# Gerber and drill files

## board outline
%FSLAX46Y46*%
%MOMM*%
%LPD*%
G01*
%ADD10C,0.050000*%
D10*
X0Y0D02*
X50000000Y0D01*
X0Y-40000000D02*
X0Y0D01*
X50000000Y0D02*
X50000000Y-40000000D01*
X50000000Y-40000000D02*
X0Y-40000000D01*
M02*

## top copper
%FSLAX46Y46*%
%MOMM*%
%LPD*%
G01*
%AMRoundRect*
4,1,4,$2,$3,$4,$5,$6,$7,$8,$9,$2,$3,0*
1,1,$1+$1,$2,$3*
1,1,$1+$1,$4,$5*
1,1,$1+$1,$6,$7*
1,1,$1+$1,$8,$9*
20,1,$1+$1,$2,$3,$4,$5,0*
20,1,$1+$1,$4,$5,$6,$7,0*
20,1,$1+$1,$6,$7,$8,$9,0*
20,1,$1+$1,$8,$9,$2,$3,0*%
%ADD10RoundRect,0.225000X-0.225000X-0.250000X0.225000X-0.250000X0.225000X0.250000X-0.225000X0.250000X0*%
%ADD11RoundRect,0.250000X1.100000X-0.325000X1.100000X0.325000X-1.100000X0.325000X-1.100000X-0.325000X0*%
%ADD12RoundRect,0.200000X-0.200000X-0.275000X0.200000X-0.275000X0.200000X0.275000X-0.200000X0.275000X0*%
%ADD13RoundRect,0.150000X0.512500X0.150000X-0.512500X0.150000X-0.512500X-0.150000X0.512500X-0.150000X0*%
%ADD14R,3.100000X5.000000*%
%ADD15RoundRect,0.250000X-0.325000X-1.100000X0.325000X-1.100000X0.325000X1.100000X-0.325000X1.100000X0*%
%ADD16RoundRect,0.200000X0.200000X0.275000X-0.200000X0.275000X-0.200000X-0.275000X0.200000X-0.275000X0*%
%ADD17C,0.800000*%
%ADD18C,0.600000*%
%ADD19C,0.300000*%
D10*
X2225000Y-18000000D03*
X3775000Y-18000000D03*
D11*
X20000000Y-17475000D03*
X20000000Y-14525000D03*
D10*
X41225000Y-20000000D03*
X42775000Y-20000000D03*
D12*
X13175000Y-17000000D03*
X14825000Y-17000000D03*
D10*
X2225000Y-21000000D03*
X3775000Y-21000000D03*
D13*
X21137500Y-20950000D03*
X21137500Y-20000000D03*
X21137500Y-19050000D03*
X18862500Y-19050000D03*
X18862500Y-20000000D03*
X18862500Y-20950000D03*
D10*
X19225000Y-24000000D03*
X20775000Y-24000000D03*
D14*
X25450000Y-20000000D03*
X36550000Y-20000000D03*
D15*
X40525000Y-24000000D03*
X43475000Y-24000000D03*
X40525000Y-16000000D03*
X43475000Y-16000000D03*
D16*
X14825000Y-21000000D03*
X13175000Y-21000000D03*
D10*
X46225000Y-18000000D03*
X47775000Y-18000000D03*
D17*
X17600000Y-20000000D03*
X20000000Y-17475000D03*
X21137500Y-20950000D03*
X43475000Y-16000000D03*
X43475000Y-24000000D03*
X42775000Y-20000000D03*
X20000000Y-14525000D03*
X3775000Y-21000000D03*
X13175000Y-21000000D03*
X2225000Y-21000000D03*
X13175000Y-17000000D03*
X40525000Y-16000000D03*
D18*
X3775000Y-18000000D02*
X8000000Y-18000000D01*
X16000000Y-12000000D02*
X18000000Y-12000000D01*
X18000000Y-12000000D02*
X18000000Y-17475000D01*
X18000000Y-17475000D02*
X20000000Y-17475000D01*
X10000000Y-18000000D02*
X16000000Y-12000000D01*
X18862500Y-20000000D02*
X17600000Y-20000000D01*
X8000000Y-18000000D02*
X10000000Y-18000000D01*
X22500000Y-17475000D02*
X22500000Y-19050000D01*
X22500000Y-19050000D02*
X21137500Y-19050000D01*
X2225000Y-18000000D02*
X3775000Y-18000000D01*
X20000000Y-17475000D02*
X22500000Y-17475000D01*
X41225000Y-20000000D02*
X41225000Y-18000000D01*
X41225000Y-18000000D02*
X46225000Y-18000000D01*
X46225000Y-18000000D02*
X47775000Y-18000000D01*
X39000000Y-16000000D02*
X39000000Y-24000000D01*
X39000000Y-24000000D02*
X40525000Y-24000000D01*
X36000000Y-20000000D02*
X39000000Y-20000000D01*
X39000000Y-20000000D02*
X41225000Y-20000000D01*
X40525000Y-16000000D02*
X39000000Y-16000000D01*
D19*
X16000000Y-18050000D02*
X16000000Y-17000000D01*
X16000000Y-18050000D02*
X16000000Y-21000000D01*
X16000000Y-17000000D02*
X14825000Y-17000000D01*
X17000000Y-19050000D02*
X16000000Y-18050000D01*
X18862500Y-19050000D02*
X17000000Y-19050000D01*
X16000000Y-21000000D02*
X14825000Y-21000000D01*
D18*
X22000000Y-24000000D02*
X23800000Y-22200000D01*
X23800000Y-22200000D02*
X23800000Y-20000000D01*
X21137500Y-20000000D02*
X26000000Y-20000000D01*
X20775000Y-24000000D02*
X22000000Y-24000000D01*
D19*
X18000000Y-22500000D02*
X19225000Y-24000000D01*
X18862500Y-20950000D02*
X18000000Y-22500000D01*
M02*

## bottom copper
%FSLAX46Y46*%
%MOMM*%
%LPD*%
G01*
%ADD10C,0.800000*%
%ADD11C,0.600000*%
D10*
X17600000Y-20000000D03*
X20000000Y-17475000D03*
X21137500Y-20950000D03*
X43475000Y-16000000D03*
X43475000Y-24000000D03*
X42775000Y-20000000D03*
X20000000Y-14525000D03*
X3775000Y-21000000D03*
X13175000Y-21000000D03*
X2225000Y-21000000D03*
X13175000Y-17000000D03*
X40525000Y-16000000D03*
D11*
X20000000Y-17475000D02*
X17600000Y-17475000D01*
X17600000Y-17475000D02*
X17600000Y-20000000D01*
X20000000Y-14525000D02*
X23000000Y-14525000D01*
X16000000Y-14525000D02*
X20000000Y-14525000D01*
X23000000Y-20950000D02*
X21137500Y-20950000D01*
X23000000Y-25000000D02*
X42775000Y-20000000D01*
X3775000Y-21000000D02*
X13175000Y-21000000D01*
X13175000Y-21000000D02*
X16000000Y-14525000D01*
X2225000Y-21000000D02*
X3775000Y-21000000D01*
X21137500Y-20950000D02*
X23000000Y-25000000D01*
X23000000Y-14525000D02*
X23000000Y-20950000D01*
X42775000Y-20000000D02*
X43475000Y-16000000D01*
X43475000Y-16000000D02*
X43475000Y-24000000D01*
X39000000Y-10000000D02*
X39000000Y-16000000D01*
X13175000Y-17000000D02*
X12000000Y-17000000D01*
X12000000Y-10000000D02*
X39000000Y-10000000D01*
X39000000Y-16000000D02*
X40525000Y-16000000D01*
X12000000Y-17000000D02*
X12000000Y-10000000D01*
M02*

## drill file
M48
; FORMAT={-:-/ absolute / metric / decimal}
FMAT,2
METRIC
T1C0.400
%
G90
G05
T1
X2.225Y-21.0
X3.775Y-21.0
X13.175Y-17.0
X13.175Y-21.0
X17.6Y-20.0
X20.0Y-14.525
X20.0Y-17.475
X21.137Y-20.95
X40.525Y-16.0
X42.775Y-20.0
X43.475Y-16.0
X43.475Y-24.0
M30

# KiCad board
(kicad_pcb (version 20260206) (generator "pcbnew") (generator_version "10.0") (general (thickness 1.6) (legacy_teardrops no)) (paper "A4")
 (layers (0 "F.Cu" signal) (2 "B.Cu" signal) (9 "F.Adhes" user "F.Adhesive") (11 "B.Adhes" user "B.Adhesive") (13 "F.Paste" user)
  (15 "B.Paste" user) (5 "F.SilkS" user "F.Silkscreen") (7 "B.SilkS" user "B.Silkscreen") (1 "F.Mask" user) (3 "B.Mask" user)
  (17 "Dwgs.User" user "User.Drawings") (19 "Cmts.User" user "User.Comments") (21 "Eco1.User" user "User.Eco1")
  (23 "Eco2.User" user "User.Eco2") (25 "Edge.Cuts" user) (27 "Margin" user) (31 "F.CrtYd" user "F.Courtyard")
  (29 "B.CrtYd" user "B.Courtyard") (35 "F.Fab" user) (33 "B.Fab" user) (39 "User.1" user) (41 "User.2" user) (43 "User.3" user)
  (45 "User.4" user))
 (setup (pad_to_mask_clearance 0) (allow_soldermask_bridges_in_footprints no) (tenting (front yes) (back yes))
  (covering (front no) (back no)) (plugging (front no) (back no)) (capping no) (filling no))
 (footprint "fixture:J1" (layer "F.Cu") (at 3 18)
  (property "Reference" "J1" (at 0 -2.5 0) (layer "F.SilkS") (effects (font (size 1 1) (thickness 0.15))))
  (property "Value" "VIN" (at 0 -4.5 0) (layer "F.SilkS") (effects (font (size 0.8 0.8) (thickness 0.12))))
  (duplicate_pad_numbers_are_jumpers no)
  (pad "1" smd roundrect (at -0.775 0) (size 0.9 0.95) (layers "F.Cu" "F.Mask" "F.Paste") (roundrect_rratio 0.25) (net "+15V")
   (thermal_bridge_angle 45))
  (pad "2" smd roundrect (at 0.775 0) (size 0.9 0.95) (layers "F.Cu" "F.Mask" "F.Paste") (roundrect_rratio 0.25) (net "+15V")
   (thermal_bridge_angle 45)))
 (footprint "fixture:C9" (layer "F.Cu") (at 20 16 90)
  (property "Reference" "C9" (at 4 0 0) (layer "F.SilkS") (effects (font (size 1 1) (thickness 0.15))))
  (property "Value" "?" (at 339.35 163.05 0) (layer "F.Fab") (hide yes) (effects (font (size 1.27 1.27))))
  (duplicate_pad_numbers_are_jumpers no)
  (pad "1" smd roundrect (at -1.475 0 90) (size 1.15 2.7) (layers "F.Cu" "F.Mask" "F.Paste") (roundrect_rratio 0.217391) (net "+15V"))
  (pad "2" smd roundrect (at 1.475 0 90) (size 1.15 2.7) (layers "F.Cu" "F.Mask" "F.Paste") (roundrect_rratio 0.217391) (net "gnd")))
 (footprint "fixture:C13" (layer "F.Cu") (at 42 20)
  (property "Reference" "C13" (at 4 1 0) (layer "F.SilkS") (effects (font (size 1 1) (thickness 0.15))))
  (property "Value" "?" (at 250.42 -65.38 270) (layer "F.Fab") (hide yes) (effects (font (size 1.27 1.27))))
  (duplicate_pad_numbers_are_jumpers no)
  (pad "1" smd roundrect (at -0.775 0) (size 0.9 0.95) (layers "F.Cu" "F.Mask" "F.Paste") (roundrect_rratio 0.25) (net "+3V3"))
  (pad "2" smd roundrect (at 0.775 0) (size 0.9 0.95) (layers "F.Cu" "F.Mask" "F.Paste") (roundrect_rratio 0.25) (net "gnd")))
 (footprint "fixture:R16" (layer "F.Cu") (at 14 17)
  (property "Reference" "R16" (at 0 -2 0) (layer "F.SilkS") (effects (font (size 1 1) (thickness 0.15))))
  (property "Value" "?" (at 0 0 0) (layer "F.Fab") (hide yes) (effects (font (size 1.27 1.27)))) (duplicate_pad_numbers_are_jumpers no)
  (pad "1" smd roundrect (at -0.825 0) (size 0.8 0.95) (layers "F.Cu" "F.Mask" "F.Paste") (roundrect_rratio 0.25) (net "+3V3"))
  (pad "2" smd roundrect (at 0.825 0) (size 0.8 0.95) (layers "F.Cu" "F.Mask" "F.Paste") (roundrect_rratio 0.25) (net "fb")))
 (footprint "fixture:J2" (layer "F.Cu") (at 3 21)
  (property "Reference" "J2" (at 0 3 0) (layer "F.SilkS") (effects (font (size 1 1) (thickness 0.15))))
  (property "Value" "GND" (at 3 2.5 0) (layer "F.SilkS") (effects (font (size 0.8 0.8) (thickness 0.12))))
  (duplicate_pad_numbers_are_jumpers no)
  (pad "1" smd roundrect (at -0.775 0) (size 0.9 0.95) (layers "F.Cu" "F.Mask" "F.Paste") (roundrect_rratio 0.25) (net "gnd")
   (thermal_bridge_angle 45))
  (pad "2" smd roundrect (at 0.775 0) (size 0.9 0.95) (layers "F.Cu" "F.Mask" "F.Paste") (roundrect_rratio 0.25) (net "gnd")
   (thermal_bridge_angle 45)))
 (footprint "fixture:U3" (layer "F.Cu") (at 20 20 180)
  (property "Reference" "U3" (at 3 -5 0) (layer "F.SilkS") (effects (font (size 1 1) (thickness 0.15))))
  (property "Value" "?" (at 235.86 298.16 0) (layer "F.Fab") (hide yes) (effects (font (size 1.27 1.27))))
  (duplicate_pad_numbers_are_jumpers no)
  (pad "1" smd roundrect (at -1.1375 -0.95 180) (size 1.325 0.6) (layers "F.Cu" "F.Mask" "F.Paste") (roundrect_rratio 0.25) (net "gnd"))
  (pad "2" smd roundrect (at -1.1375 0 180) (size 1.325 0.6) (layers "F.Cu" "F.Mask" "F.Paste") (roundrect_rratio 0.25) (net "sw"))
  (pad "3" smd roundrect (at -1.1375 0.95 180) (size 1.325 0.6) (layers "F.Cu" "F.Mask" "F.Paste") (roundrect_rratio 0.25) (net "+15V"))
  (pad "4" smd roundrect (at 1.1375 0.95 180) (size 1.325 0.6) (layers "F.Cu" "F.Mask" "F.Paste") (roundrect_rratio 0.25) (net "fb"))
  (pad "5" smd roundrect (at 1.1375 0 180) (size 1.325 0.6) (layers "F.Cu" "F.Mask" "F.Paste") (roundrect_rratio 0.25) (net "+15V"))
  (pad "6" smd roundrect (at 1.1375 -0.95 180) (size 1.325 0.6) (layers "F.Cu" "F.Mask" "F.Paste") (roundrect_rratio 0.25) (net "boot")))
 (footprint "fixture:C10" (layer "F.Cu") (at 20 24)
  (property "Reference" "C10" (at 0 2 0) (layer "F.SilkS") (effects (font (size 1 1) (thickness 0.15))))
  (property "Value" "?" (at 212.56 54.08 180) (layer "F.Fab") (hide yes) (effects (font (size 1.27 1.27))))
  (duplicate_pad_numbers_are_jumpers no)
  (pad "1" smd roundrect (at -0.775 0) (size 0.9 0.95) (layers "F.Cu" "F.Mask" "F.Paste") (roundrect_rratio 0.25) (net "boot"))
  (pad "2" smd roundrect (at 0.775 0) (size 0.9 0.95) (layers "F.Cu" "F.Mask" "F.Paste") (roundrect_rratio 0.25) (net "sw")))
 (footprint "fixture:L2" (layer "F.Cu") (at 31 20)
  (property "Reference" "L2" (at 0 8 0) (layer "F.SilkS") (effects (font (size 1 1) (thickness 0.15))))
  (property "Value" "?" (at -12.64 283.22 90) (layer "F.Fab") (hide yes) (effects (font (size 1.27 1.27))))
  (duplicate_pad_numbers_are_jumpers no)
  (pad "1" smd rect (at -5.55 0) (size 3.1 5) (layers "F.Cu" "F.Mask" "F.Paste") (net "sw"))
  (pad "2" smd rect (at 5.55 0) (size 3.1 5) (layers "F.Cu" "F.Mask" "F.Paste") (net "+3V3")))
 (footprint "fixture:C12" (layer "F.Cu") (at 42 24)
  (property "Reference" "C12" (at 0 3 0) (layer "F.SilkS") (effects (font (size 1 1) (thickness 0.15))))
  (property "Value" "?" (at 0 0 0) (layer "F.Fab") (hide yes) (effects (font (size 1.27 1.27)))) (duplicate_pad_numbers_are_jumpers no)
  (pad "1" smd roundrect (at -1.475 0) (size 1.15 2.7) (layers "F.Cu" "F.Mask" "F.Paste") (roundrect_rratio 0.217391) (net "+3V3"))
  (pad "2" smd roundrect (at 1.475 0) (size 1.15 2.7) (layers "F.Cu" "F.Mask" "F.Paste") (roundrect_rratio 0.217391) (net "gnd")))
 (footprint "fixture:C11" (layer "F.Cu") (at 42 16)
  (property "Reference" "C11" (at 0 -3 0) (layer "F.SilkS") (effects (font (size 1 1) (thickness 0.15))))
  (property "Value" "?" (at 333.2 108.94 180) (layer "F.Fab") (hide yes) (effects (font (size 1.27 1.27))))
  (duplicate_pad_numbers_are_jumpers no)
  (pad "1" smd roundrect (at -1.475 0) (size 1.15 2.7) (layers "F.Cu" "F.Mask" "F.Paste") (roundrect_rratio 0.217391) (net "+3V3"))
  (pad "2" smd roundrect (at 1.475 0) (size 1.15 2.7) (layers "F.Cu" "F.Mask" "F.Paste") (roundrect_rratio 0.217391) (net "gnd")))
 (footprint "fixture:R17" (layer "F.Cu") (at 14 21 180)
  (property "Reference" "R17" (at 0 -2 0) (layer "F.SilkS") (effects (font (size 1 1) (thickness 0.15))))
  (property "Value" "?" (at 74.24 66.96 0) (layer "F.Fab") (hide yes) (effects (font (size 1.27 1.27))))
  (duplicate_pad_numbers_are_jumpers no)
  (pad "1" smd roundrect (at -0.825 0 180) (size 0.8 0.95) (layers "F.Cu" "F.Mask" "F.Paste") (roundrect_rratio 0.25) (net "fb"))
  (pad "2" smd roundrect (at 0.825 0 180) (size 0.8 0.95) (layers "F.Cu" "F.Mask" "F.Paste") (roundrect_rratio 0.25) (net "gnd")))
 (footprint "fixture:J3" (layer "F.Cu") (at 47 18)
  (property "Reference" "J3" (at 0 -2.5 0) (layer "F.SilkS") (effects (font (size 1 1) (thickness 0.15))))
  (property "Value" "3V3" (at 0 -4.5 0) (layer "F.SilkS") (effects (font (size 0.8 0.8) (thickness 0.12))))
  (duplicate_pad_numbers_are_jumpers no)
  (pad "1" smd roundrect (at -0.775 0) (size 0.9 0.95) (layers "F.Cu" "F.Mask" "F.Paste") (roundrect_rratio 0.25) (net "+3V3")
   (thermal_bridge_angle 45))
  (pad "2" smd roundrect (at 0.775 0) (size 0.9 0.95) (layers "F.Cu" "F.Mask" "F.Paste") (roundrect_rratio 0.25) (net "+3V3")
   (thermal_bridge_angle 45)))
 (gr_line (start 0 0) (end 50 0) (stroke (width 0.05) (type default)) (layer "Edge.Cuts"))
 (gr_line (start 0 40) (end 0 0) (stroke (width 0.05) (type default)) (layer "Edge.Cuts"))
 (gr_line (start 50 0) (end 50 40) (stroke (width 0.05) (type default)) (layer "Edge.Cuts"))
 (gr_line (start 50 40) (end 0 40) (stroke (width 0.05) (type default)) (layer "Edge.Cuts"))
 (segment (start 3.775 18) (end 8 18) (width 0.6) (layer "F.Cu") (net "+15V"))
 (segment (start 16 12) (end 18 12) (width 0.6) (layer "F.Cu") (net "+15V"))
 (segment (start 18 12) (end 18 17.475) (width 0.6) (layer "F.Cu") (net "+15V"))
 (segment (start 18 17.475) (end 20 17.475) (width 0.6) (layer "F.Cu") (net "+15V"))
 (segment (start 10 18) (end 16 12) (width 0.6) (layer "F.Cu") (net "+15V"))
 (segment (start 18.8625 20) (end 17.6 20) (width 0.6) (layer "F.Cu") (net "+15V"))
 (segment (start 8 18) (end 10 18) (width 0.6) (layer "F.Cu") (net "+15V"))
 (segment (start 22.5 17.475) (end 22.5 19.05) (width 0.6) (layer "F.Cu") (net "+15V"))
 (segment (start 22.5 19.05) (end 21.1375 19.05) (width 0.6) (layer "F.Cu") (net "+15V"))
 (segment (start 2.225 18) (end 3.775 18) (width 0.6) (layer "F.Cu") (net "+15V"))
 (segment (start 20 17.475) (end 22.5 17.475) (width 0.6) (layer "F.Cu") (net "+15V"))
 (via (at 17.6 20) (size 0.8) (drill 0.4) (layers "F.Cu" "B.Cu") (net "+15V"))
 (via (at 20 17.475) (size 0.8) (drill 0.4) (layers "F.Cu" "B.Cu") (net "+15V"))
 (segment (start 20 17.475) (end 17.6 17.475) (width 0.6) (layer "B.Cu") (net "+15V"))
 (segment (start 17.6 17.475) (end 17.6 20) (width 0.6) (layer "B.Cu") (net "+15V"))
 (via (at 21.1375 20.95) (size 0.8) (drill 0.4) (layers "F.Cu" "B.Cu") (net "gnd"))
 (via (at 43.475 16) (size 0.8) (drill 0.4) (layers "F.Cu" "B.Cu") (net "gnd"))
 (via (at 43.475 24) (size 0.8) (drill 0.4) (layers "F.Cu" "B.Cu") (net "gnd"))
 (via (at 42.775 20) (size 0.8) (drill 0.4) (layers "F.Cu" "B.Cu") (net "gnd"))
 (via (at 20 14.525) (size 0.8) (drill 0.4) (layers "F.Cu" "B.Cu") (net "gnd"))
 (via (at 3.775 21) (size 0.8) (drill 0.4) (layers "F.Cu" "B.Cu") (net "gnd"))
 (via (at 13.175 21) (size 0.8) (drill 0.4) (layers "F.Cu" "B.Cu") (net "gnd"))
 (via (at 2.225 21) (size 0.8) (drill 0.4) (layers "F.Cu" "B.Cu") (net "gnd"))
 (segment (start 20 14.525) (end 23 14.525) (width 0.6) (layer "B.Cu") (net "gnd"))
 (segment (start 16 14.525) (end 20 14.525) (width 0.6) (layer "B.Cu") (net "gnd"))
 (segment (start 23 20.95) (end 21.1375 20.95) (width 0.6) (layer "B.Cu") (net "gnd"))
 (segment (start 23 25) (end 42.775 20) (width 0.6) (layer "B.Cu") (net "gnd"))
 (segment (start 3.775 21) (end 13.175 21) (width 0.6) (layer "B.Cu") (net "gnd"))
 (segment (start 13.175 21) (end 16 14.525) (width 0.6) (layer "B.Cu") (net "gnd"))
 (segment (start 2.225 21) (end 3.775 21) (width 0.6) (layer "B.Cu") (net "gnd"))
 (segment (start 21.1375 20.95) (end 23 25) (width 0.6) (layer "B.Cu") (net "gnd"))
 (segment (start 23 14.525) (end 23 20.95) (width 0.6) (layer "B.Cu") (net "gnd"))
 (segment (start 42.775 20) (end 43.475 16) (width 0.6) (layer "B.Cu") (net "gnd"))
 (segment (start 43.475 16) (end 43.475 24) (width 0.6) (layer "B.Cu") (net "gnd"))
 (segment (start 41.225 20) (end 41.225 18) (width 0.6) (layer "F.Cu") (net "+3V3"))
 (segment (start 41.225 18) (end 46.225 18) (width 0.6) (layer "F.Cu") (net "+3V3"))
 (segment (start 46.225 18) (end 47.775 18) (width 0.6) (layer "F.Cu") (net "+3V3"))
 (segment (start 39 16) (end 39 24) (width 0.6) (layer "F.Cu") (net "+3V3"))
 (segment (start 39 24) (end 40.525 24) (width 0.6) (layer "F.Cu") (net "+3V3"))
 (segment (start 36 20) (end 39 20) (width 0.6) (layer "F.Cu") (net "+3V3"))
 (segment (start 39 20) (end 41.225 20) (width 0.6) (layer "F.Cu") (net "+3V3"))
 (segment (start 40.525 16) (end 39 16) (width 0.6) (layer "F.Cu") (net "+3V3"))
 (via (at 13.175 17) (size 0.8) (drill 0.4) (layers "F.Cu" "B.Cu") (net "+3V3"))
 (via (at 40.525 16) (size 0.8) (drill 0.4) (layers "F.Cu" "B.Cu") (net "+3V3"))
 (segment (start 39 10) (end 39 16) (width 0.6) (layer "B.Cu") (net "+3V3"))
 (segment (start 13.175 17) (end 12 17) (width 0.6) (layer "B.Cu") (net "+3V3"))
 (segment (start 12 10) (end 39 10) (width 0.6) (layer "B.Cu") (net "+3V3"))
 (segment (start 39 16) (end 40.525 16) (width 0.6) (layer "B.Cu") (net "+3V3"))
 (segment (start 12 17) (end 12 10) (width 0.6) (layer "B.Cu") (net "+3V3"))
 (segment (start 16 18.05) (end 16 17) (width 0.3) (layer "F.Cu") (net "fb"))
 (segment (start 16 18.05) (end 16 21) (width 0.3) (layer "F.Cu") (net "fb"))
 (segment (start 16 17) (end 14.825 17) (width 0.3) (layer "F.Cu") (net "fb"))
 (segment (start 17 19.05) (end 16 18.05) (width 0.3) (layer "F.Cu") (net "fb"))
 (segment (start 18.8625 19.05) (end 17 19.05) (width 0.3) (layer "F.Cu") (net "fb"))
 (segment (start 16 21) (end 14.825 21) (width 0.3) (layer "F.Cu") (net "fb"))
 (segment (start 22 24) (end 23.8 22.2) (width 0.6) (layer "F.Cu") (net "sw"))
 (segment (start 23.8 22.2) (end 23.8 20) (width 0.6) (layer "F.Cu") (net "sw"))
 (segment (start 21.1375 20) (end 26 20) (width 0.6) (layer "F.Cu") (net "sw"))
 (segment (start 20.775 24) (end 22 24) (width 0.6) (layer "F.Cu") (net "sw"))
 (segment (start 18 22.5) (end 19.225 24) (width 0.3) (layer "F.Cu") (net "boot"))
 (segment (start 18.8625 20.95) (end 18 22.5) (width 0.3) (layer "F.Cu") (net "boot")))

